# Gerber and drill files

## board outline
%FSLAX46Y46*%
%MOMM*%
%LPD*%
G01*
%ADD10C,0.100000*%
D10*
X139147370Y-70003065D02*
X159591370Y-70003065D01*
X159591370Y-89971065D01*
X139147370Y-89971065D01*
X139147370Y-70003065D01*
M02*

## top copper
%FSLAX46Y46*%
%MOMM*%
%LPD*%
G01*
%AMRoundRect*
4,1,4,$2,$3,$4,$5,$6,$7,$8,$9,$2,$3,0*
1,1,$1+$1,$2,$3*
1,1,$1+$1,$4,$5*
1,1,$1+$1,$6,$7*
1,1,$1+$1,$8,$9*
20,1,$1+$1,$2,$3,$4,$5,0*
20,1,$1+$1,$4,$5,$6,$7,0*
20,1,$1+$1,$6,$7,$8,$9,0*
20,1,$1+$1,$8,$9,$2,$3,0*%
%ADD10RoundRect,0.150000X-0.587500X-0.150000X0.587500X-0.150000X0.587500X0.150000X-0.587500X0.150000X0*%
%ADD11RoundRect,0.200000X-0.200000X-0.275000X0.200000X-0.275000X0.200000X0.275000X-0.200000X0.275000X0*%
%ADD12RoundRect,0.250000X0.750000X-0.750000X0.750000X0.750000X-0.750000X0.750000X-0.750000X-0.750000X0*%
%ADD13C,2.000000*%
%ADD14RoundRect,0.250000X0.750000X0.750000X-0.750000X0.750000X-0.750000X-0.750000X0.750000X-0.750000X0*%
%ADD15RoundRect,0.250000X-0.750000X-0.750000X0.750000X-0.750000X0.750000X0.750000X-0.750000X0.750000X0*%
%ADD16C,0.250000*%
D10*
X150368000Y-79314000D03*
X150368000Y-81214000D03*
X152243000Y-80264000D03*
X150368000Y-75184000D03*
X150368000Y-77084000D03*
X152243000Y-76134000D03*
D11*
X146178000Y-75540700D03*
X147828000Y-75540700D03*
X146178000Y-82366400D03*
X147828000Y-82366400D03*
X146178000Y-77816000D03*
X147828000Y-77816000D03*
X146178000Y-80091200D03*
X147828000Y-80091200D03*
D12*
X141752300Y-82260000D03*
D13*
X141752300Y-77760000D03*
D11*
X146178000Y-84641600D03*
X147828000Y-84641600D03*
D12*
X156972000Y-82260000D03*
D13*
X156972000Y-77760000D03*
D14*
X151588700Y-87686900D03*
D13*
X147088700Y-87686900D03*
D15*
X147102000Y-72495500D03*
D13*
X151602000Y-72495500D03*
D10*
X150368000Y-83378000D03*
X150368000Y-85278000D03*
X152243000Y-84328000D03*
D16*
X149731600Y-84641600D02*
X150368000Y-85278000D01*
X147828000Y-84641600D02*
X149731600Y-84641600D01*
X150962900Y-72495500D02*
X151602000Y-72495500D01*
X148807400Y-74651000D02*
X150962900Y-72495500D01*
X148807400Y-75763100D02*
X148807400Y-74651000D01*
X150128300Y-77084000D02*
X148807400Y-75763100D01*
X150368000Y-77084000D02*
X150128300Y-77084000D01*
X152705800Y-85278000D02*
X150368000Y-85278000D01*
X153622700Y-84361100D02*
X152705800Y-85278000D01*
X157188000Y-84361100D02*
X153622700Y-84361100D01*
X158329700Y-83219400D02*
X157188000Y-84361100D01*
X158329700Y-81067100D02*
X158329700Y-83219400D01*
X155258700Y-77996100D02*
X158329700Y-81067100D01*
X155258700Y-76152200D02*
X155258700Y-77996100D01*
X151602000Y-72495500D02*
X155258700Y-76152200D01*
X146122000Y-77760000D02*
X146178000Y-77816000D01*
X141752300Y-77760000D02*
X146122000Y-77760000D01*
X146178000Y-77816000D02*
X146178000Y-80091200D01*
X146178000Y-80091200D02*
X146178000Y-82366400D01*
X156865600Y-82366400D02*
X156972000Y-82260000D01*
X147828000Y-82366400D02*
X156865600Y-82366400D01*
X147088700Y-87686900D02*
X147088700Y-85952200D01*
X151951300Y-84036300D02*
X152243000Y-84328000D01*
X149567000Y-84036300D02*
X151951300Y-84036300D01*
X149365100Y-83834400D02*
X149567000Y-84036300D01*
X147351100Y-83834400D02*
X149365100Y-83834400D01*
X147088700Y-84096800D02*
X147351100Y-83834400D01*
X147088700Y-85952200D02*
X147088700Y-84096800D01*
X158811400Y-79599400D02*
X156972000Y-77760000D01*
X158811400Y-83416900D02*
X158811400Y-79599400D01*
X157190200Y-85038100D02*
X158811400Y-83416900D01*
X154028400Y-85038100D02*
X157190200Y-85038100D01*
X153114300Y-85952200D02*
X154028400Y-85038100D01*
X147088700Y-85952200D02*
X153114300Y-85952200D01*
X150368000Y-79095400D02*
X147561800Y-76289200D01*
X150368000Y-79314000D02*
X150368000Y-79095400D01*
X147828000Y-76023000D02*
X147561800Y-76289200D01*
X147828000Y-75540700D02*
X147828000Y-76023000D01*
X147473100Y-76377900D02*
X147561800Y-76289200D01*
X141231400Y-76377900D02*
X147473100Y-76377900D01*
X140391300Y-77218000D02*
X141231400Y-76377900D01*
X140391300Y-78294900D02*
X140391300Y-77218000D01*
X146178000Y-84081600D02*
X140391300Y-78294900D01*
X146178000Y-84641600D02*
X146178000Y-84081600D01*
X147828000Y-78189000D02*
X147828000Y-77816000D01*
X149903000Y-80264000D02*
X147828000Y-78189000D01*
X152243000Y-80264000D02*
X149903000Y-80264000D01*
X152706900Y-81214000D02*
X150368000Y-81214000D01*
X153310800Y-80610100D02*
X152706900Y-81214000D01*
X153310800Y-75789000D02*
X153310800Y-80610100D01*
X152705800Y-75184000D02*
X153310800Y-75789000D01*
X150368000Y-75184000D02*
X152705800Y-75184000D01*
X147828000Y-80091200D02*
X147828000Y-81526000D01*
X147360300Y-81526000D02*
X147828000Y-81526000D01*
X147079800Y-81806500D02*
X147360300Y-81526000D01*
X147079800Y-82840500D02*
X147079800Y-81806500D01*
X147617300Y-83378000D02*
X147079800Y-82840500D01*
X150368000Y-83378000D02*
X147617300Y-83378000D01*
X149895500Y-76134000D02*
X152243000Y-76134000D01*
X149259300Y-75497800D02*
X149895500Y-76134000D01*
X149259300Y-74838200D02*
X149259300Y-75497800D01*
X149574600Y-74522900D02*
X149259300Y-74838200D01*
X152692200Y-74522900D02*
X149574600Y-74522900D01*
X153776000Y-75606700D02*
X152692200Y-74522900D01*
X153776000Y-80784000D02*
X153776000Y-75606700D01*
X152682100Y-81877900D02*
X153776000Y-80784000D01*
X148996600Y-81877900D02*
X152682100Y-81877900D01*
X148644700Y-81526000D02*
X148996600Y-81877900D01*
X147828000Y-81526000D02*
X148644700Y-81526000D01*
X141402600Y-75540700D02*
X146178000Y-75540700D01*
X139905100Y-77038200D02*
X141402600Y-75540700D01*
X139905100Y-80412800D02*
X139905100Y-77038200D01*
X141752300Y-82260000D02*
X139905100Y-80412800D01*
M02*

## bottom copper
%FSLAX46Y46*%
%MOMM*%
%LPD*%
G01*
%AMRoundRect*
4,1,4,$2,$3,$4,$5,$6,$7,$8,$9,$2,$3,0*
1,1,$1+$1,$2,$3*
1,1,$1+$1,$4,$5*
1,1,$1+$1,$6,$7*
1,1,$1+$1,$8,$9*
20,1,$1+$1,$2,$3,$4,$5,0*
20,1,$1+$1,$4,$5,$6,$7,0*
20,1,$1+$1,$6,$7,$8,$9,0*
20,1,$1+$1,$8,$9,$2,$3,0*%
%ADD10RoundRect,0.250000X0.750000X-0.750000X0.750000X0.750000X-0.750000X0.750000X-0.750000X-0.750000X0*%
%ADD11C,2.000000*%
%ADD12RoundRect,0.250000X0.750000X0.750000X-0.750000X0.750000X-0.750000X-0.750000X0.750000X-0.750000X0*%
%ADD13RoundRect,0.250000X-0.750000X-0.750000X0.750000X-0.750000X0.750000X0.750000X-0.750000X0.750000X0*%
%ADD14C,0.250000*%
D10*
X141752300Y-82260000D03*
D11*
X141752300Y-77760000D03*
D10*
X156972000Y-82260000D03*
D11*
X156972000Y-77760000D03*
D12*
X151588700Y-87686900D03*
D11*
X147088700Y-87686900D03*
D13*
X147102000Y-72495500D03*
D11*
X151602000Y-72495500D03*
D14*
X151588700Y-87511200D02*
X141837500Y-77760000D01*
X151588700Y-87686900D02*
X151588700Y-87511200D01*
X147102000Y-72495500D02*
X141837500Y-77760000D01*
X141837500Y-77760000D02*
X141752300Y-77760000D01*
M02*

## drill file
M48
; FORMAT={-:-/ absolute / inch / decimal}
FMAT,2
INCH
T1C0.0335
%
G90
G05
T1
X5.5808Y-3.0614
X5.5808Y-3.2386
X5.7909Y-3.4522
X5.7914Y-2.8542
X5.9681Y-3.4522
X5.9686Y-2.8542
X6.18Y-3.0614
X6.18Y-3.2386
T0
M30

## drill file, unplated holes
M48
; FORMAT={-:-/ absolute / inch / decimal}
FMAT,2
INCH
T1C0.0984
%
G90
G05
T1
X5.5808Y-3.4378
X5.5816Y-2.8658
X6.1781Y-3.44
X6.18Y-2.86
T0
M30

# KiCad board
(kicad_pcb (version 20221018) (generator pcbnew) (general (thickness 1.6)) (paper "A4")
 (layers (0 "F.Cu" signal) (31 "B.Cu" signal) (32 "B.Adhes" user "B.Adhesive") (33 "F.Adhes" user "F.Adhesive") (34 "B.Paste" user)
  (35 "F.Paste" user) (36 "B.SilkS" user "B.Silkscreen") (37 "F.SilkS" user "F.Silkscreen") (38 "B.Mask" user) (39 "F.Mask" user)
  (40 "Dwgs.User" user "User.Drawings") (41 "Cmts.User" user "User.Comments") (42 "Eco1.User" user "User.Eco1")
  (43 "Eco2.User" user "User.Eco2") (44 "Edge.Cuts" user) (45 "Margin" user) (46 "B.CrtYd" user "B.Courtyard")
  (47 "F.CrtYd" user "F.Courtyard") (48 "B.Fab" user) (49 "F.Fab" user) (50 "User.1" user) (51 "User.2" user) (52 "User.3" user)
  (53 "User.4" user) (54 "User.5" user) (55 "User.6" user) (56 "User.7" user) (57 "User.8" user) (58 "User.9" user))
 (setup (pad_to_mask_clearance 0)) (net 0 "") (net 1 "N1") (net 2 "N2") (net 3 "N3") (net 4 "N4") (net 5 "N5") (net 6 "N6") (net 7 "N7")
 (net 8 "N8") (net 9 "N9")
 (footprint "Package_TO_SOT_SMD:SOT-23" (layer "F.Cu") (at 151.3055 80.264)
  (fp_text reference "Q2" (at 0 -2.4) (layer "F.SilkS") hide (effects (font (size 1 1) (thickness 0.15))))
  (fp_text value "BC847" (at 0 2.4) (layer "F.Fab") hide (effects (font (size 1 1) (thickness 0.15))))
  (pad "1" smd roundrect (at -0.9375 -0.95) (size 1.475 0.6) (layers "F.Cu" "F.Paste" "F.Mask") (roundrect_rratio 0.25) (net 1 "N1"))
  (pad "2" smd roundrect (at -0.9375 0.95) (size 1.475 0.6) (layers "F.Cu" "F.Paste" "F.Mask") (roundrect_rratio 0.25) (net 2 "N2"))
  (pad "3" smd roundrect (at 0.9375 0) (size 1.475 0.6) (layers "F.Cu" "F.Paste" "F.Mask") (roundrect_rratio 0.25) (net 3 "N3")))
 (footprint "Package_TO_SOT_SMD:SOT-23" (layer "F.Cu") (at 151.3055 76.134)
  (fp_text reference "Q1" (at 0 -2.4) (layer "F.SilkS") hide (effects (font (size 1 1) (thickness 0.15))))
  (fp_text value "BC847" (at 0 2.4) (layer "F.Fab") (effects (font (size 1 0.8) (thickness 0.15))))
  (pad "1" smd roundrect (at -0.9375 -0.95) (size 1.475 0.6) (layers "F.Cu" "F.Paste" "F.Mask") (roundrect_rratio 0.25) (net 2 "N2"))
  (pad "2" smd roundrect (at -0.9375 0.95) (size 1.475 0.6) (layers "F.Cu" "F.Paste" "F.Mask") (roundrect_rratio 0.25) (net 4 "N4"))
  (pad "3" smd roundrect (at 0.9375 0) (size 1.475 0.6) (layers "F.Cu" "F.Paste" "F.Mask") (roundrect_rratio 0.25) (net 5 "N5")))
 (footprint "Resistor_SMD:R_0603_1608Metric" (layer "F.Cu") (at 147.003 75.5407)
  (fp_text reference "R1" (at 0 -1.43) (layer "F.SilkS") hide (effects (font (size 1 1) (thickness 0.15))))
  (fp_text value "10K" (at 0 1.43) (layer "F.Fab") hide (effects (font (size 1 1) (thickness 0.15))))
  (pad "1" smd roundrect (at -0.825 0) (size 0.8 0.95) (layers "F.Cu" "F.Paste" "F.Mask") (roundrect_rratio 0.25) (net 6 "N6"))
  (pad "2" smd roundrect (at 0.825 0) (size 0.8 0.95) (layers "F.Cu" "F.Paste" "F.Mask") (roundrect_rratio 0.25) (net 1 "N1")))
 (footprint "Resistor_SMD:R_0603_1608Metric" (layer "F.Cu") (at 147.003 82.3664)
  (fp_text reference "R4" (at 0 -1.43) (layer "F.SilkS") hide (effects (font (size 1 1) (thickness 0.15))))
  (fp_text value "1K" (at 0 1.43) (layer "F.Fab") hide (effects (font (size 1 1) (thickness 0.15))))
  (pad "1" smd roundrect (at -0.825 0) (size 0.8 0.95) (layers "F.Cu" "F.Paste" "F.Mask") (roundrect_rratio 0.25) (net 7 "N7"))
  (pad "2" smd roundrect (at 0.825 0) (size 0.8 0.95) (layers "F.Cu" "F.Paste" "F.Mask") (roundrect_rratio 0.25) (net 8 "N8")))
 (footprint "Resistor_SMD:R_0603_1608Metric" (layer "F.Cu") (at 147.003 77.816)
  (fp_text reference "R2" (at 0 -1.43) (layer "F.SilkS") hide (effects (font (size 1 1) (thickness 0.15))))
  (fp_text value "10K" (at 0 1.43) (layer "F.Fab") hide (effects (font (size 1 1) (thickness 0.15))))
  (pad "1" smd roundrect (at -0.825 0) (size 0.8 0.95) (layers "F.Cu" "F.Paste" "F.Mask") (roundrect_rratio 0.25) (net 7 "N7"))
  (pad "2" smd roundrect (at 0.825 0) (size 0.8 0.95) (layers "F.Cu" "F.Paste" "F.Mask") (roundrect_rratio 0.25) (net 3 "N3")))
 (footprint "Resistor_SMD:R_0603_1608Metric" (layer "F.Cu") (at 147.003 80.0912)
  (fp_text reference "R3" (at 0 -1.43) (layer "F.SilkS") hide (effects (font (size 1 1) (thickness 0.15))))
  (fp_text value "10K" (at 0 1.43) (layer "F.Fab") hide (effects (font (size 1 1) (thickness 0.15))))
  (pad "1" smd roundrect (at -0.825 0) (size 0.8 0.95) (layers "F.Cu" "F.Paste" "F.Mask") (roundrect_rratio 0.25) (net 7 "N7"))
  (pad "2" smd roundrect (at 0.825 0) (size 0.8 0.95) (layers "F.Cu" "F.Paste" "F.Mask") (roundrect_rratio 0.25) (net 5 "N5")))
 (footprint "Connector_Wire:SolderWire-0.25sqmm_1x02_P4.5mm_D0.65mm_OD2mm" (layer "F.Cu") (at 141.7523 82.26 90)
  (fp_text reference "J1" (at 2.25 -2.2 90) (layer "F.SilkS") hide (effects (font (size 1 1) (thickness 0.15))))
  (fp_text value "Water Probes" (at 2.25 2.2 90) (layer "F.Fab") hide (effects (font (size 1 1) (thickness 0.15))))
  (pad "1" thru_hole roundrect (at 0 0 90) (size 2 2) (drill 0.85) (layers "*.Cu" "*.Mask") (roundrect_rratio 0.125) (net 6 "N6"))
  (pad "2" thru_hole circle (at 4.5 0 90) (size 2 2) (drill 0.85) (layers "*.Cu" "*.Mask") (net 7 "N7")))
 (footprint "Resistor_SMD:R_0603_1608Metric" (layer "F.Cu") (at 147.003 84.6416)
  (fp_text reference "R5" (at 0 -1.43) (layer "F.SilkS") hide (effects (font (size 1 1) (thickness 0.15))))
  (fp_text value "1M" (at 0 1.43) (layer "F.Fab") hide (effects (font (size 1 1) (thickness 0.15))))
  (pad "1" smd roundrect (at -0.825 0) (size 0.8 0.95) (layers "F.Cu" "F.Paste" "F.Mask") (roundrect_rratio 0.25) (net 1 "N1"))
  (pad "2" smd roundrect (at 0.825 0) (size 0.8 0.95) (layers "F.Cu" "F.Paste" "F.Mask") (roundrect_rratio 0.25) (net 4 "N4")))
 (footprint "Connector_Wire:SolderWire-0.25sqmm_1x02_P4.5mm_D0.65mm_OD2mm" (layer "F.Cu") (at 156.972 82.26 90)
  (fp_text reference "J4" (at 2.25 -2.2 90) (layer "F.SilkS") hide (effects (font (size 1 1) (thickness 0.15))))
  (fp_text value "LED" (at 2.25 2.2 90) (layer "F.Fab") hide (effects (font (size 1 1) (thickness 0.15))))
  (pad "1" thru_hole roundrect (at 0 0 90) (size 2 2) (drill 0.85) (layers "*.Cu" "*.Mask") (roundrect_rratio 0.125) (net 8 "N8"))
  (pad "2" thru_hole circle (at 4.5 0 90) (size 2 2) (drill 0.85) (layers "*.Cu" "*.Mask") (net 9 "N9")))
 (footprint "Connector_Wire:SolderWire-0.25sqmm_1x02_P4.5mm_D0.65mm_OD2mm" (layer "F.Cu") (at 151.5887 87.6869 180)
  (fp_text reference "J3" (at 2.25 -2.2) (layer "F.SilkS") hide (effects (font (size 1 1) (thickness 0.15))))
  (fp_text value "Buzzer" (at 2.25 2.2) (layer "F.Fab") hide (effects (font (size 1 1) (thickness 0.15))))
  (pad "1" thru_hole roundrect (at 0 0 180) (size 2 2) (drill 0.85) (layers "*.Cu" "*.Mask") (roundrect_rratio 0.125) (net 7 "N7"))
  (pad "2" thru_hole circle (at 4.5 0 180) (size 2 2) (drill 0.85) (layers "*.Cu" "*.Mask") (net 9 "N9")))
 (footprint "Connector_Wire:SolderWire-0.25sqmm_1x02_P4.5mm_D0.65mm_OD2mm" (layer "F.Cu") (at 147.102 72.4955)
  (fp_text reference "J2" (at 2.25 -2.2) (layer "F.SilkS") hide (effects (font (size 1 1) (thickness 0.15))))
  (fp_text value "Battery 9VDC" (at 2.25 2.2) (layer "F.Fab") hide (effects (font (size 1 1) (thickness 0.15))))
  (pad "1" thru_hole roundrect (at 0 0) (size 2 2) (drill 0.85) (layers "*.Cu" "*.Mask") (roundrect_rratio 0.125) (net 7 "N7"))
  (pad "2" thru_hole circle (at 4.5 0) (size 2 2) (drill 0.85) (layers "*.Cu" "*.Mask") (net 4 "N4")))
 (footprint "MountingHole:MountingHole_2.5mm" (layer "F.Cu") (at 156.925 87.376)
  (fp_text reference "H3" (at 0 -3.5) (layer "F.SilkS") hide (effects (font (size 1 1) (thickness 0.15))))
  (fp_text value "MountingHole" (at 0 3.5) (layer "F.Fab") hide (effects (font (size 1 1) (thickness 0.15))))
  (pad "" np_thru_hole circle (at 0 0) (size 2.5 2.5) (drill 2.5) (layers "*.Cu" "*.Mask")))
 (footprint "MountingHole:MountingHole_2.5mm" (layer "F.Cu") (at 141.7523 87.3191)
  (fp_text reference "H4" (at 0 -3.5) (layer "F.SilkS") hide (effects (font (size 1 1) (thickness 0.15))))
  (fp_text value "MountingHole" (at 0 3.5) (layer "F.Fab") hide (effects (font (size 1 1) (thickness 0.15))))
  (pad "" np_thru_hole circle (at 0 0) (size 2.5 2.5) (drill 2.5) (layers "*.Cu" "*.Mask")))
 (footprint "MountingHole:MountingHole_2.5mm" (layer "F.Cu") (at 141.7726 72.7925)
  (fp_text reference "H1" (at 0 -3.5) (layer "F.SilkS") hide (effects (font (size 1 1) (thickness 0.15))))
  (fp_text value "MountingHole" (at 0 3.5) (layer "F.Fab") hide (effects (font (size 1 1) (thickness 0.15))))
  (pad "" np_thru_hole circle (at 0 0) (size 2.5 2.5) (drill 2.5) (layers "*.Cu" "*.Mask")))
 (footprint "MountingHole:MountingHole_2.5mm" (layer "F.Cu") (at 156.972 72.644)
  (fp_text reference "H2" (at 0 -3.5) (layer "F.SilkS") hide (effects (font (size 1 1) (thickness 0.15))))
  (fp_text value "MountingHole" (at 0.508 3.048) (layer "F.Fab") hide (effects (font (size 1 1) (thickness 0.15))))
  (pad "" np_thru_hole circle (at 0 0) (size 2.5 2.5) (drill 2.5) (layers "*.Cu" "*.Mask")))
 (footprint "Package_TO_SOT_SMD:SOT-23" (layer "F.Cu") (at 151.3055 84.328)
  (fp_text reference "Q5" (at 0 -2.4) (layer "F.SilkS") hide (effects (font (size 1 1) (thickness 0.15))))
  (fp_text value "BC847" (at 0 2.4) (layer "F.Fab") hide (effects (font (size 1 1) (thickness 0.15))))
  (pad "1" smd roundrect (at -0.9375 -0.95) (size 1.475 0.6) (layers "F.Cu" "F.Paste" "F.Mask") (roundrect_rratio 0.25) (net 5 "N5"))
  (pad "2" smd roundrect (at -0.9375 0.95) (size 1.475 0.6) (layers "F.Cu" "F.Paste" "F.Mask") (roundrect_rratio 0.25) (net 4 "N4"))
  (pad "3" smd roundrect (at 0.9375 0) (size 1.475 0.6) (layers "F.Cu" "F.Paste" "F.Mask") (roundrect_rratio 0.25) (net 9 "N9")))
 (gr_rect (start 139.14737 70.003065) (end 159.59137 89.971065) (stroke (width 0.1) (type default)) (fill none) (layer "Edge.Cuts"))
 (segment (start 139.9051 80.4128) (end 139.9051 77.0382) (width 0.25) (layer "F.Cu") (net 6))
 (segment (start 139.9051 77.0382) (end 141.4026 75.5407) (width 0.25) (layer "F.Cu") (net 6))
 (segment (start 141.4026 75.5407) (end 146.178 75.5407) (width 0.25) (layer "F.Cu") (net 6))
 (segment (start 141.7523 82.26) (end 139.9051 80.4128) (width 0.25) (layer "F.Cu") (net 6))
 (segment (start 148.6447 81.526) (end 148.9966 81.8779) (width 0.25) (layer "F.Cu") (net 5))
 (segment (start 153.776 75.6067) (end 152.6922 74.5229) (width 0.25) (layer "F.Cu") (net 5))
 (segment (start 147.828 81.526) (end 148.6447 81.526) (width 0.25) (layer "F.Cu") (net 5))
 (segment (start 149.2593 75.4978) (end 149.8955 76.134) (width 0.25) (layer "F.Cu") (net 5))
 (segment (start 147.6173 83.378) (end 147.0798 82.8405) (width 0.25) (layer "F.Cu") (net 5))
 (segment (start 147.828 80.0912) (end 147.828 81.526) (width 0.25) (layer "F.Cu") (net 5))
 (segment (start 147.0798 82.8405) (end 147.0798 81.8065) (width 0.25) (layer "F.Cu") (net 5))
 (segment (start 150.368 83.378) (end 147.6173 83.378) (width 0.25) (layer "F.Cu") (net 5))
 (segment (start 149.2593 74.8382) (end 149.2593 75.4978) (width 0.25) (layer "F.Cu") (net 5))
 (segment (start 149.5746 74.5229) (end 149.2593 74.8382) (width 0.25) (layer "F.Cu") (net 5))
 (segment (start 152.6922 74.5229) (end 149.5746 74.5229) (width 0.25) (layer "F.Cu") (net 5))
 (segment (start 147.0798 81.8065) (end 147.3603 81.526) (width 0.25) (layer "F.Cu") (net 5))
 (segment (start 152.6821 81.8779) (end 153.776 80.784) (width 0.25) (layer "F.Cu") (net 5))
 (segment (start 148.9966 81.8779) (end 152.6821 81.8779) (width 0.25) (layer "F.Cu") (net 5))
 (segment (start 153.776 80.784) (end 153.776 75.6067) (width 0.25) (layer "F.Cu") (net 5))
 (segment (start 149.8955 76.134) (end 152.243 76.134) (width 0.25) (layer "F.Cu") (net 5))
 (segment (start 147.3603 81.526) (end 147.828 81.526) (width 0.25) (layer "F.Cu") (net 5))
 (segment (start 150.368 75.184) (end 152.7058 75.184) (width 0.25) (layer "F.Cu") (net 2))
 (segment (start 152.7058 75.184) (end 153.3108 75.789) (width 0.25) (layer "F.Cu") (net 2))
 (segment (start 153.3108 75.789) (end 153.3108 80.6101) (width 0.25) (layer "F.Cu") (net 2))
 (segment (start 153.3108 80.6101) (end 152.7069 81.214) (width 0.25) (layer "F.Cu") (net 2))
 (segment (start 152.7069 81.214) (end 150.368 81.214) (width 0.25) (layer "F.Cu") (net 2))
 (segment (start 152.243 80.264) (end 149.903 80.264) (width 0.25) (layer "F.Cu") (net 3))
 (segment (start 147.828 78.189) (end 147.828 77.816) (width 0.25) (layer "F.Cu") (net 3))
 (segment (start 149.903 80.264) (end 147.828 78.189) (width 0.25) (layer "F.Cu") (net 3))
 (segment (start 150.368 79.0954) (end 147.5618 76.2892) (width 0.25) (layer "F.Cu") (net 1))
 (segment (start 147.828 76.023) (end 147.5618 76.2892) (width 0.25) (layer "F.Cu") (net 1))
 (segment (start 146.178 84.6416) (end 146.178 84.0816) (width 0.25) (layer "F.Cu") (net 1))
 (segment (start 147.828 75.5407) (end 147.828 76.023) (width 0.25) (layer "F.Cu") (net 1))
 (segment (start 146.178 84.0816) (end 140.3913 78.2949) (width 0.25) (layer "F.Cu") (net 1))
 (segment (start 150.368 79.314) (end 150.368 79.0954) (width 0.25) (layer "F.Cu") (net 1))
 (segment (start 147.4731 76.3779) (end 147.5618 76.2892) (width 0.25) (layer "F.Cu") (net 1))
 (segment (start 140.3913 78.2949) (end 140.3913 77.218) (width 0.25) (layer "F.Cu") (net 1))
 (segment (start 140.3913 77.218) (end 141.2314 76.3779) (width 0.25) (layer "F.Cu") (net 1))
 (segment (start 141.2314 76.3779) (end 147.4731 76.3779) (width 0.25) (layer "F.Cu") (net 1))
 (segment (start 158.8114 79.5994) (end 156.972 77.76) (width 0.25) (layer "F.Cu") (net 9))
 (segment (start 149.567 84.0363) (end 151.9513 84.0363) (width 0.25) (layer "F.Cu") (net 9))
 (segment (start 149.3651 83.8344) (end 149.567 84.0363) (width 0.25) (layer "F.Cu") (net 9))
 (segment (start 147.3511 83.8344) (end 149.3651 83.8344) (width 0.25) (layer "F.Cu") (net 9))
 (segment (start 153.1143 85.9522) (end 154.0284 85.0381) (width 0.25) (layer "F.Cu") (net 9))
 (segment (start 151.9513 84.0363) (end 152.243 84.328) (width 0.25) (layer "F.Cu") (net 9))
 (segment (start 154.0284 85.0381) (end 157.1902 85.0381) (width 0.25) (layer "F.Cu") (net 9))
 (segment (start 147.0887 84.0968) (end 147.3511 83.8344) (width 0.25) (layer "F.Cu") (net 9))
 (segment (start 147.0887 85.9522) (end 153.1143 85.9522) (width 0.25) (layer "F.Cu") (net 9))
 (segment (start 147.0887 87.6869) (end 147.0887 85.9522) (width 0.25) (layer "F.Cu") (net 9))
 (segment (start 157.1902 85.0381) (end 158.8114 83.4169) (width 0.25) (layer "F.Cu") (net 9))
 (segment (start 147.0887 85.9522) (end 147.0887 84.0968) (width 0.25) (layer "F.Cu") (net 9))
 (segment (start 158.8114 83.4169) (end 158.8114 79.5994) (width 0.25) (layer "F.Cu") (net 9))
 (segment (start 147.828 82.3664) (end 156.8656 82.3664) (width 0.25) (layer "F.Cu") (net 8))
 (segment (start 156.8656 82.3664) (end 156.972 82.26) (width 0.25) (layer "F.Cu") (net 8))
 (segment (start 146.122 77.76) (end 146.178 77.816) (width 0.25) (layer "F.Cu") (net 7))
 (segment (start 146.178 77.816) (end 146.178 80.0912) (width 0.25) (layer "F.Cu") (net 7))
 (segment (start 141.7523 77.76) (end 146.122 77.76) (width 0.25) (layer "F.Cu") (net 7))
 (segment (start 146.178 80.0912) (end 146.178 82.3664) (width 0.25) (layer "F.Cu") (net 7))
 (segment (start 141.8375 77.76) (end 141.7523 77.76) (width 0.25) (layer "B.Cu") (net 7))
 (segment (start 151.5887 87.5112) (end 141.8375 77.76) (width 0.25) (layer "B.Cu") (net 7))
 (segment (start 151.5887 87.6869) (end 151.5887 87.5112) (width 0.25) (layer "B.Cu") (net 7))
 (segment (start 147.102 72.4955) (end 141.8375 77.76) (width 0.25) (layer "B.Cu") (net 7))
 (segment (start 157.188 84.3611) (end 153.6227 84.3611) (width 0.25) (layer "F.Cu") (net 4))
 (segment (start 148.8074 74.651) (end 150.9629 72.4955) (width 0.25) (layer "F.Cu") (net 4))
 (segment (start 158.3297 83.2194) (end 157.188 84.3611) (width 0.25) (layer "F.Cu") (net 4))
 (segment (start 150.368 77.084) (end 150.1283 77.084) (width 0.25) (layer "F.Cu") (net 4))
 (segment (start 150.9629 72.4955) (end 151.602 72.4955) (width 0.25) (layer "F.Cu") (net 4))
 (segment (start 155.2587 77.9961) (end 158.3297 81.0671) (width 0.25) (layer "F.Cu") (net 4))
 (segment (start 151.602 72.4955) (end 155.2587 76.1522) (width 0.25) (layer "F.Cu") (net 4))
 (segment (start 155.2587 76.1522) (end 155.2587 77.9961) (width 0.25) (layer "F.Cu") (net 4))
 (segment (start 153.6227 84.3611) (end 152.7058 85.278) (width 0.25) (layer "F.Cu") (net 4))
 (segment (start 158.3297 81.0671) (end 158.3297 83.2194) (width 0.25) (layer "F.Cu") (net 4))
 (segment (start 147.828 84.6416) (end 149.7316 84.6416) (width 0.25) (layer "F.Cu") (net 4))
 (segment (start 148.8074 75.7631) (end 148.8074 74.651) (width 0.25) (layer "F.Cu") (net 4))
 (segment (start 149.7316 84.6416) (end 150.368 85.278) (width 0.25) (layer "F.Cu") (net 4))
 (segment (start 150.1283 77.084) (end 148.8074 75.7631) (width 0.25) (layer "F.Cu") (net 4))
 (segment (start 152.7058 85.278) (end 150.368 85.278) (width 0.25) (layer "F.Cu") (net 4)))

